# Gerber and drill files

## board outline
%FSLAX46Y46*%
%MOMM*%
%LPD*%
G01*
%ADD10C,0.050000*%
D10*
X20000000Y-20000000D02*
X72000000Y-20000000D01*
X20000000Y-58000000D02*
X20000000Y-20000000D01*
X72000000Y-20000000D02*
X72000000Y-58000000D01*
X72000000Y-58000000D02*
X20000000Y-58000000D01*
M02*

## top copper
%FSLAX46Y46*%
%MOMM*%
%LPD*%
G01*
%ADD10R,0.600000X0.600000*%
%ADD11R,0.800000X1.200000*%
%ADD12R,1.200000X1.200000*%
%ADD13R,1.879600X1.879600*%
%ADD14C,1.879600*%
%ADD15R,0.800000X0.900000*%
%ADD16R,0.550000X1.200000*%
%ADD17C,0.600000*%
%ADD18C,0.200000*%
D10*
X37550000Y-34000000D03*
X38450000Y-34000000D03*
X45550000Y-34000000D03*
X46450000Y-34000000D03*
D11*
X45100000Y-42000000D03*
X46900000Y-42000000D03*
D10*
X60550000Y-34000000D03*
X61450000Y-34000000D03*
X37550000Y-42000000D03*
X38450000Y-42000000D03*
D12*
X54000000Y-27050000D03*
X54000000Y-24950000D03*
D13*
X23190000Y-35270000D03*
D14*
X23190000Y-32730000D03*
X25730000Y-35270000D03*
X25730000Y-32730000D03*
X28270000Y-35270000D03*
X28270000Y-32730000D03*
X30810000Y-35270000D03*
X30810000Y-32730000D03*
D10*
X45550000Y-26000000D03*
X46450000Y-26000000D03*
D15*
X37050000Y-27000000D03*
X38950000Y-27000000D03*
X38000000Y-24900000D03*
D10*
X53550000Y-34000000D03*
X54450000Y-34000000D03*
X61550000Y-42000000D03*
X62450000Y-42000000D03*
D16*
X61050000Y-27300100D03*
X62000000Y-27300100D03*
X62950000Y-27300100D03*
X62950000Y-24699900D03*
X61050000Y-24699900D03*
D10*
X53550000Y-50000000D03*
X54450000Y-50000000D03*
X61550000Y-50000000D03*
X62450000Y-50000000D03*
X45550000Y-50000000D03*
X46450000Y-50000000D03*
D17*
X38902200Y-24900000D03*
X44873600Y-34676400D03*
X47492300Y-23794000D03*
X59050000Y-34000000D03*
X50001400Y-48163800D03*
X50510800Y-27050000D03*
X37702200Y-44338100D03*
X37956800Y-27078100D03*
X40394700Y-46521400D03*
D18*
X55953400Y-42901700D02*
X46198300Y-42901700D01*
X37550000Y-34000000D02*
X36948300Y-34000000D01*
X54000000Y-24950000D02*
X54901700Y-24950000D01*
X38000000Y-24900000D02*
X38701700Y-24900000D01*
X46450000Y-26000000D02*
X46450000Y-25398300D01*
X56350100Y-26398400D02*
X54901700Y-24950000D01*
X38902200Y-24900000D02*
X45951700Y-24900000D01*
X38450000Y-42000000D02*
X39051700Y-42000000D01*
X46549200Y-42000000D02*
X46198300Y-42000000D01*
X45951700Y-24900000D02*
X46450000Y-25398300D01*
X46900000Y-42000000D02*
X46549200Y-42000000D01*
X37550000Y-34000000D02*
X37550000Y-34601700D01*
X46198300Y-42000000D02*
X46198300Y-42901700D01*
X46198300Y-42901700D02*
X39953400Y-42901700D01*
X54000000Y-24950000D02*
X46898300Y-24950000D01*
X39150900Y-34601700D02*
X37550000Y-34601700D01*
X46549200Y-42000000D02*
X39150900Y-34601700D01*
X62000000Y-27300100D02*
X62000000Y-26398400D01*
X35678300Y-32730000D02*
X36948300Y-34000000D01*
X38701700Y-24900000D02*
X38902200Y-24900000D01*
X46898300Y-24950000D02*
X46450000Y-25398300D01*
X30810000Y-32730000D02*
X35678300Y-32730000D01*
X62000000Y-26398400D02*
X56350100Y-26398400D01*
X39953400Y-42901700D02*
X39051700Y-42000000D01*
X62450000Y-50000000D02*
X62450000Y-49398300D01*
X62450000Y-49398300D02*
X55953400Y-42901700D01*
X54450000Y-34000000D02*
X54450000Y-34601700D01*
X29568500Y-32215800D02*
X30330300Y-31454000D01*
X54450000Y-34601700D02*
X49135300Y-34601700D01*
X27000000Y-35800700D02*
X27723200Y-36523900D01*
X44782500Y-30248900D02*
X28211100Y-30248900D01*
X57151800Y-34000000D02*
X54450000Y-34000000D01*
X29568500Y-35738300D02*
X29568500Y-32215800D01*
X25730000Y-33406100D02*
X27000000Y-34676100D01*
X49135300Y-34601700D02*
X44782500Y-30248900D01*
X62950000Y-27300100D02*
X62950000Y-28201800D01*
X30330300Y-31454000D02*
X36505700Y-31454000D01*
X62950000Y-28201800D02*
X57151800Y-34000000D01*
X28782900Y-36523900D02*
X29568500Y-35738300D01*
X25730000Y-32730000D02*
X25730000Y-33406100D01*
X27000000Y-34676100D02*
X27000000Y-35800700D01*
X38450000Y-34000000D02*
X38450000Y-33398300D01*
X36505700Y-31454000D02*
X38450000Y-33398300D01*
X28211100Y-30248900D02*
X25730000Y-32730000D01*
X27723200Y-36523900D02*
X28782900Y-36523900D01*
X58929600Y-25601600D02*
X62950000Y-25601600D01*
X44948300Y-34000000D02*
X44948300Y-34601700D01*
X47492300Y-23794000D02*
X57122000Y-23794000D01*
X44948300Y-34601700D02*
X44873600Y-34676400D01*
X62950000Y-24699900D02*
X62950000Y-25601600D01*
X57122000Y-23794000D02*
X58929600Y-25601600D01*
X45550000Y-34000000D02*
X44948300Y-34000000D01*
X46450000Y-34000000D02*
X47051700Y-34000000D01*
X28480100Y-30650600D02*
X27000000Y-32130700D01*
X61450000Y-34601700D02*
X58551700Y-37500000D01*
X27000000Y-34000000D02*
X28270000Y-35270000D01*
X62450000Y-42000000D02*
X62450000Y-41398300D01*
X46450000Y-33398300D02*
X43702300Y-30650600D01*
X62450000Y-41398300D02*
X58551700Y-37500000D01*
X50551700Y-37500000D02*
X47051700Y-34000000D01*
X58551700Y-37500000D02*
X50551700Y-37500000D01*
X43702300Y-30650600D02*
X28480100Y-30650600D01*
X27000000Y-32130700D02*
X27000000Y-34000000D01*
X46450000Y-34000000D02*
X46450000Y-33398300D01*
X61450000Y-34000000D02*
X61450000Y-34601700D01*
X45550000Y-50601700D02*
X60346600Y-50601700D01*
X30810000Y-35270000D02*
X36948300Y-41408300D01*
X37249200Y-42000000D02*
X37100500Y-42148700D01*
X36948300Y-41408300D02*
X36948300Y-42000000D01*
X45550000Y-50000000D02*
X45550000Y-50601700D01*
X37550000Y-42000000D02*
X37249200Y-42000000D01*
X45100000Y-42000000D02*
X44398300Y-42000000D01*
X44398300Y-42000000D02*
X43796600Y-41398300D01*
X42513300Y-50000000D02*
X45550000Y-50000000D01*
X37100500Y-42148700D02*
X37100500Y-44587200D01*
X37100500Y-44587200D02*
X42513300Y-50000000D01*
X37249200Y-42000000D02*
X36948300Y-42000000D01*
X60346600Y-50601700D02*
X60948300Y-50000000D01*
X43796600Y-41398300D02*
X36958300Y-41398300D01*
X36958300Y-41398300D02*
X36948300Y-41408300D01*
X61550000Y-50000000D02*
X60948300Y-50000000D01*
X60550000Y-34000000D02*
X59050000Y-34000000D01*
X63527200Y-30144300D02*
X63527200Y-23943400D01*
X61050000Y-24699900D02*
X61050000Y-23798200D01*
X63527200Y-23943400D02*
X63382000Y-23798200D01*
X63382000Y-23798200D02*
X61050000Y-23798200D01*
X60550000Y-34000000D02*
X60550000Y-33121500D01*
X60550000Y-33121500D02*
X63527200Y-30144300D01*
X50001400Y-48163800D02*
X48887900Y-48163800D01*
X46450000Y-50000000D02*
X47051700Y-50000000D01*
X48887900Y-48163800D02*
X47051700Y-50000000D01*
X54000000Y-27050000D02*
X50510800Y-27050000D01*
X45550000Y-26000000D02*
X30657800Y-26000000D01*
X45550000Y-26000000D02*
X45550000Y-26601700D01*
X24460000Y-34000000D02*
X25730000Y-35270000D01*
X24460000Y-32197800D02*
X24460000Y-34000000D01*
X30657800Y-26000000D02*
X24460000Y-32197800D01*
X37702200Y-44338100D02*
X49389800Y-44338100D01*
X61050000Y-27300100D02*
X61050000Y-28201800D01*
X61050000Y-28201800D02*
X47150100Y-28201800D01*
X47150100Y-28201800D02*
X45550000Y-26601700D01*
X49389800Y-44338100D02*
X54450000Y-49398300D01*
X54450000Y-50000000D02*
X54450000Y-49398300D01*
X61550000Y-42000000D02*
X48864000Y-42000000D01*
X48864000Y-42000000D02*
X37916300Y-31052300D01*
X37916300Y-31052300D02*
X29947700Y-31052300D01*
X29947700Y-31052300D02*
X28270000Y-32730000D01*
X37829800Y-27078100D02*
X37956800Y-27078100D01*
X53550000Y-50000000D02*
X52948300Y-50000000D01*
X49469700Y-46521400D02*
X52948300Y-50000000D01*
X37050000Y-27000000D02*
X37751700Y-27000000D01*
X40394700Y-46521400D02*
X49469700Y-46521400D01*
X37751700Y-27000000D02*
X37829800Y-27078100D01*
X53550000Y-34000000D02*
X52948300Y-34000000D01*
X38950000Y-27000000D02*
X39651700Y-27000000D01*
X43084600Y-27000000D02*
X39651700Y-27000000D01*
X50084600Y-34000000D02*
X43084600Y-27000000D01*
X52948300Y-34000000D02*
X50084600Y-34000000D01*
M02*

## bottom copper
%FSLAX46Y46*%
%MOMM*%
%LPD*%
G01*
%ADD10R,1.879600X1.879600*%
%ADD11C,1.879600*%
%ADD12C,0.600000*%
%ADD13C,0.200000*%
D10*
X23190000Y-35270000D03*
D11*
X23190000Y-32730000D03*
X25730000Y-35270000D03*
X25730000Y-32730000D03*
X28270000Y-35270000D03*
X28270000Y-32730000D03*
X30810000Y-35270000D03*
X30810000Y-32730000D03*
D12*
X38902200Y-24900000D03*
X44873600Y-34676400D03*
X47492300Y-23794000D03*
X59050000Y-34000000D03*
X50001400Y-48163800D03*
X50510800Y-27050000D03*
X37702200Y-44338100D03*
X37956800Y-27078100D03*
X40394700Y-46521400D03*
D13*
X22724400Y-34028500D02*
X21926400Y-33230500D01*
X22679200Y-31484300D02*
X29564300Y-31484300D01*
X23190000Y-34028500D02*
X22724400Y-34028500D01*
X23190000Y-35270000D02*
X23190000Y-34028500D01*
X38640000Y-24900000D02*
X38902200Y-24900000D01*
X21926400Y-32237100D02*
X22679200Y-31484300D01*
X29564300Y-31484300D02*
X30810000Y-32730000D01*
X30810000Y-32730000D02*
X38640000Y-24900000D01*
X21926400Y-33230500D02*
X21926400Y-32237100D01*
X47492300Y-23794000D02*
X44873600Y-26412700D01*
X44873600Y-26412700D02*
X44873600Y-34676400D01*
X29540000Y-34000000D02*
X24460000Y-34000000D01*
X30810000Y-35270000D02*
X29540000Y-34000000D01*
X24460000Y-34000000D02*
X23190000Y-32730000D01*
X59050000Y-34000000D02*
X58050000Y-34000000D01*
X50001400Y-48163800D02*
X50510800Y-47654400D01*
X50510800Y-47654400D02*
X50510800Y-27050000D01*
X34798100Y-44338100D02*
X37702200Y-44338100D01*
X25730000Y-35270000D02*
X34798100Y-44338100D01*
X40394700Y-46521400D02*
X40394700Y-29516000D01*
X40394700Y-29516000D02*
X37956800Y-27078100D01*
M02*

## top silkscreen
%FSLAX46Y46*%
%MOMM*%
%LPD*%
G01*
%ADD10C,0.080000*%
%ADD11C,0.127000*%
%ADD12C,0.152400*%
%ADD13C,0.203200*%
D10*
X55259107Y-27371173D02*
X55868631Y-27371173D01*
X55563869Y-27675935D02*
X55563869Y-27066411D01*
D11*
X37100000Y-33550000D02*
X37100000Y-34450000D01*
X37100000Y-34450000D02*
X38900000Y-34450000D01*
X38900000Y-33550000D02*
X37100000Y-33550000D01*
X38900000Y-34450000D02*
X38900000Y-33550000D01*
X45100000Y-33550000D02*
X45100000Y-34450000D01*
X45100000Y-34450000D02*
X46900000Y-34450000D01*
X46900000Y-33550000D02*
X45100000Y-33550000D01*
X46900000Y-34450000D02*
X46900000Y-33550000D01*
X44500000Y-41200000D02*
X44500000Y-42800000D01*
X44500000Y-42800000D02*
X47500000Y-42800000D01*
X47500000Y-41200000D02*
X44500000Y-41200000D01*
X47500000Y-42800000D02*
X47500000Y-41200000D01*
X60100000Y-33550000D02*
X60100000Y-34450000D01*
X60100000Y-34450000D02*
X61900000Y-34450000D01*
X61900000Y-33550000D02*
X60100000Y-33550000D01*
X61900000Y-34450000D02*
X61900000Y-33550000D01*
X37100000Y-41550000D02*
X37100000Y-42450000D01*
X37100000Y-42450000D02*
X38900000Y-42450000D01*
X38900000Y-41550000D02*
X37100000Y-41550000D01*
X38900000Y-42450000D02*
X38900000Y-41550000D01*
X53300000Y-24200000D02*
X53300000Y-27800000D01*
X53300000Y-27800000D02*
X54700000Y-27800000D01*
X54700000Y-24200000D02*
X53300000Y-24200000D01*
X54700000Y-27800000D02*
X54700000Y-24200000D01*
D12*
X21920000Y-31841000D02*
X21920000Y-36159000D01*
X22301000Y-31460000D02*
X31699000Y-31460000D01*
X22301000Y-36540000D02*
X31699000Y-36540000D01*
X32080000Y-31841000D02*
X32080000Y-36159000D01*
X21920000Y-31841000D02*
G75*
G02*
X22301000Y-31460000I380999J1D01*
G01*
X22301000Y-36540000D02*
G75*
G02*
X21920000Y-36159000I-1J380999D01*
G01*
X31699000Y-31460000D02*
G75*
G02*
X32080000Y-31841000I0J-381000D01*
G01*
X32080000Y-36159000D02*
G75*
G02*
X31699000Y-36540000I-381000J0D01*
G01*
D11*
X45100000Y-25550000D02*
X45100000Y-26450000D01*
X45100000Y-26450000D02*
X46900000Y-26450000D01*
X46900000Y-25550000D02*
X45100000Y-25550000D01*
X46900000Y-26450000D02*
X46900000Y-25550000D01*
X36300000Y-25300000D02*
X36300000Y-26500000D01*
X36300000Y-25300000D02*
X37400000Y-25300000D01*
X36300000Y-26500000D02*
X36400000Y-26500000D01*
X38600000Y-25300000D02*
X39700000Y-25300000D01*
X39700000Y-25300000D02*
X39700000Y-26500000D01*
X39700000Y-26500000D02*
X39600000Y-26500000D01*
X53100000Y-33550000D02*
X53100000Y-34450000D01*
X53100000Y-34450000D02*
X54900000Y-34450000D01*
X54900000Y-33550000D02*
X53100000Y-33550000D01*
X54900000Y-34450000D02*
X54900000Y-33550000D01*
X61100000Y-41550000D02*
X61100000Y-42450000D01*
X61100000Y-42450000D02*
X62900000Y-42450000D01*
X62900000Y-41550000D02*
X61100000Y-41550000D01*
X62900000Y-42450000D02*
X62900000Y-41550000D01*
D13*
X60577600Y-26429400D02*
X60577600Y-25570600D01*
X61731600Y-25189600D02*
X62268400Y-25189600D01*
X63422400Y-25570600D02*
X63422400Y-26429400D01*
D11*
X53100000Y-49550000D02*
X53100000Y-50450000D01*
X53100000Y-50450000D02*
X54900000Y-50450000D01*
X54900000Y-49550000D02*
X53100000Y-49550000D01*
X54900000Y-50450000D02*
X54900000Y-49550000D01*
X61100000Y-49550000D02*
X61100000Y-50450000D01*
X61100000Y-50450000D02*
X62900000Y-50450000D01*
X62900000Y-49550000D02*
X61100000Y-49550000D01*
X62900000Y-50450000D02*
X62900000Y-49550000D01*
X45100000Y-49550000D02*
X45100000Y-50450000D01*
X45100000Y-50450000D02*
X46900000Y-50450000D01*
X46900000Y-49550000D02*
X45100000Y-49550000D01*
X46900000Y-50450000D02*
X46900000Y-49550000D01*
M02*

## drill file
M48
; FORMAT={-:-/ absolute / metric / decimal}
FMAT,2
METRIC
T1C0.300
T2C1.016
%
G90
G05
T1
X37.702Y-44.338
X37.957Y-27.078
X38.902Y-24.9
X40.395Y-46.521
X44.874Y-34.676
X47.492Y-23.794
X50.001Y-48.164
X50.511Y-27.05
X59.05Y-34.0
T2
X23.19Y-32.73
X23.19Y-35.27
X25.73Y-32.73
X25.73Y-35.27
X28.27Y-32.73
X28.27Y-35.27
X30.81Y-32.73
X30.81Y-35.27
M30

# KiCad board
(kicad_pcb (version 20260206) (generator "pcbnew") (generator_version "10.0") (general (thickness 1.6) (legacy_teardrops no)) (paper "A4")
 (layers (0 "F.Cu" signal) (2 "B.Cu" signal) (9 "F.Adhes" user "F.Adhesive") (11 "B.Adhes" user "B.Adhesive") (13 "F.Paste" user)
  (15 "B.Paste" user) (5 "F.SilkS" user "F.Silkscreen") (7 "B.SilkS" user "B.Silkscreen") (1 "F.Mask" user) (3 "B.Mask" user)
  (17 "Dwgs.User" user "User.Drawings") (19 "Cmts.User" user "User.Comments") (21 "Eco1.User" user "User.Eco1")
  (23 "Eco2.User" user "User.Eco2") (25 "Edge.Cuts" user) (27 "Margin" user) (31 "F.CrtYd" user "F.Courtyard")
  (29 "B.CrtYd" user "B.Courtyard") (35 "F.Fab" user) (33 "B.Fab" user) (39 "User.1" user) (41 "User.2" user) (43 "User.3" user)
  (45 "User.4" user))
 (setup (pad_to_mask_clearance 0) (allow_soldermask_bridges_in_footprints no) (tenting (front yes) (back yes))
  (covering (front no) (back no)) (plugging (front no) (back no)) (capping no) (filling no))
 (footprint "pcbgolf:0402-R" (layer "F.Cu") (at 38 34)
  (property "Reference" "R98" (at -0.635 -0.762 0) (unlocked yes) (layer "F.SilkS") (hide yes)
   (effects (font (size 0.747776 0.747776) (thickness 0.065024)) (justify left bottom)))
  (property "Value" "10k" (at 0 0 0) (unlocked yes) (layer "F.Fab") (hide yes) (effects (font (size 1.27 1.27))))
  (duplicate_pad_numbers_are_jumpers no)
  (fp_line (start -0.9 -0.45) (end -0.9 0.45) (stroke (width 0.127) (type solid)) (layer "F.SilkS"))
  (fp_line (start -0.9 0.45) (end 0.9 0.45) (stroke (width 0.127) (type solid)) (layer "F.SilkS"))
  (fp_line (start 0.9 -0.45) (end -0.9 -0.45) (stroke (width 0.127) (type solid)) (layer "F.SilkS"))
  (fp_line (start 0.9 0.45) (end 0.9 -0.45) (stroke (width 0.127) (type solid)) (layer "F.SilkS"))
  (pad "1" smd rect (at -0.45 0) (size 0.6 0.6) (layers "F.Cu" "F.Mask" "F.Paste") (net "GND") (solder_mask_margin 0.0508)
   (solder_paste_margin 0) (thermal_bridge_angle 0))
  (pad "2" smd rect (at 0.45 0) (size 0.6 0.6) (layers "F.Cu" "F.Mask" "F.Paste") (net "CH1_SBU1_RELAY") (solder_mask_margin 0.0508)
   (solder_paste_margin 0) (thermal_bridge_angle 0)))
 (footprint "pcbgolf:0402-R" (layer "F.Cu") (at 46 34)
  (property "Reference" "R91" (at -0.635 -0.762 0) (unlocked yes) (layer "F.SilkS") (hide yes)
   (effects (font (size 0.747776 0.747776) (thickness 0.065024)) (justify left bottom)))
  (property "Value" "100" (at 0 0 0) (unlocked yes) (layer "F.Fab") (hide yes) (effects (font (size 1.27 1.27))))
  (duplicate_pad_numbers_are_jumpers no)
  (fp_line (start -0.9 -0.45) (end -0.9 0.45) (stroke (width 0.127) (type solid)) (layer "F.SilkS"))
  (fp_line (start -0.9 0.45) (end 0.9 0.45) (stroke (width 0.127) (type solid)) (layer "F.SilkS"))
  (fp_line (start 0.9 -0.45) (end -0.9 -0.45) (stroke (width 0.127) (type solid)) (layer "F.SilkS"))
  (fp_line (start 0.9 0.45) (end 0.9 -0.45) (stroke (width 0.127) (type solid)) (layer "F.SilkS"))
  (pad "1" smd rect (at -0.45 0) (size 0.6 0.6) (layers "F.Cu" "F.Mask" "F.Paste") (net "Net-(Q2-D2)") (solder_mask_margin 0.0508)
   (solder_paste_margin 0) (thermal_bridge_angle 0))
  (pad "2" smd rect (at 0.45 0) (size 0.6 0.6) (layers "F.Cu" "F.Mask" "F.Paste") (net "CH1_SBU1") (solder_mask_margin 0.0508)
   (solder_paste_margin 0) (thermal_bridge_angle 0)))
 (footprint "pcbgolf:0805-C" (layer "F.Cu") (at 46 42)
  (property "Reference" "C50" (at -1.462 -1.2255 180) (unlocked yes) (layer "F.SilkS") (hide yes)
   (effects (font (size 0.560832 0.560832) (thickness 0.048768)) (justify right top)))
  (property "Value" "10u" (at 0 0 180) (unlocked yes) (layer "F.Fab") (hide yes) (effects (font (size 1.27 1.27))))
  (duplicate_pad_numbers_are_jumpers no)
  (fp_line (start -1.5 -0.8) (end -1.5 0.8) (stroke (width 0.127) (type solid)) (layer "F.SilkS"))
  (fp_line (start -1.5 0.8) (end 1.5 0.8) (stroke (width 0.127) (type solid)) (layer "F.SilkS"))
  (fp_line (start 1.5 -0.8) (end -1.5 -0.8) (stroke (width 0.127) (type solid)) (layer "F.SilkS"))
  (fp_line (start 1.5 0.8) (end 1.5 -0.8) (stroke (width 0.127) (type solid)) (layer "F.SilkS"))
  (pad "1" smd rect (at -0.9 0) (size 0.8 1.2) (layers "F.Cu" "F.Mask" "F.Paste") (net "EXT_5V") (solder_mask_margin 0.0508)
   (solder_paste_margin 0) (thermal_bridge_angle 0))
  (pad "2" smd rect (at 0.9 0) (size 0.8 1.2) (layers "F.Cu" "F.Mask" "F.Paste") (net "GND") (solder_mask_margin 0.0508)
   (solder_paste_margin 0) (thermal_bridge_angle 0)))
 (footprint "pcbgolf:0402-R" (layer "F.Cu") (at 61 34)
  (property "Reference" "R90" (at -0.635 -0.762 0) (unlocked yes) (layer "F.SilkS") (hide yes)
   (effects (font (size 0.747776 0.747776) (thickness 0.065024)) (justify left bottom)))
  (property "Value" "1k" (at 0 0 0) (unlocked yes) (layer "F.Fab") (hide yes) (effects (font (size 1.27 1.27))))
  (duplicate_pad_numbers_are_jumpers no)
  (fp_line (start -0.9 -0.45) (end -0.9 0.45) (stroke (width 0.127) (type solid)) (layer "F.SilkS"))
  (fp_line (start -0.9 0.45) (end 0.9 0.45) (stroke (width 0.127) (type solid)) (layer "F.SilkS"))
  (fp_line (start 0.9 -0.45) (end -0.9 -0.45) (stroke (width 0.127) (type solid)) (layer "F.SilkS"))
  (fp_line (start 0.9 0.45) (end 0.9 -0.45) (stroke (width 0.127) (type solid)) (layer "F.SilkS"))
  (pad "1" smd rect (at -0.45 0) (size 0.6 0.6) (layers "F.Cu" "F.Mask" "F.Paste") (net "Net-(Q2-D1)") (solder_mask_margin 0.0508)
   (solder_paste_margin 0) (thermal_bridge_angle 0))
  (pad "2" smd rect (at 0.45 0) (size 0.6 0.6) (layers "F.Cu" "F.Mask" "F.Paste") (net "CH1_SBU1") (solder_mask_margin 0.0508)
   (solder_paste_margin 0) (thermal_bridge_angle 0)))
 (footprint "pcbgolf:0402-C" (layer "F.Cu") (at 38 42)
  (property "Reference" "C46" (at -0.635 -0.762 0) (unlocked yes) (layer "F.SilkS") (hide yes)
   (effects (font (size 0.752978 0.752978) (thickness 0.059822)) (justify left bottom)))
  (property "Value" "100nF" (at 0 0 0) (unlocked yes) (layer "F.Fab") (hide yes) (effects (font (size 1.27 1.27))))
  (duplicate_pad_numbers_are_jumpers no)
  (fp_line (start -0.9 -0.45) (end -0.9 0.45) (stroke (width 0.127) (type solid)) (layer "F.SilkS"))
  (fp_line (start -0.9 0.45) (end 0.9 0.45) (stroke (width 0.127) (type solid)) (layer "F.SilkS"))
  (fp_line (start 0.9 -0.45) (end -0.9 -0.45) (stroke (width 0.127) (type solid)) (layer "F.SilkS"))
  (fp_line (start 0.9 0.45) (end 0.9 -0.45) (stroke (width 0.127) (type solid)) (layer "F.SilkS"))
  (pad "1" smd rect (at -0.45 0) (size 0.6 0.6) (layers "F.Cu" "F.Mask" "F.Paste") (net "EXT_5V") (solder_mask_margin 0.0508)
   (solder_paste_margin 0) (thermal_bridge_angle 0))
  (pad "2" smd rect (at 0.45 0) (size 0.6 0.6) (layers "F.Cu" "F.Mask" "F.Paste") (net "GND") (solder_mask_margin 0.0508)
   (solder_paste_margin 0) (thermal_bridge_angle 0)))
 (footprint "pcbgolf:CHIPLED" (layer "F.Cu") (at 54 26)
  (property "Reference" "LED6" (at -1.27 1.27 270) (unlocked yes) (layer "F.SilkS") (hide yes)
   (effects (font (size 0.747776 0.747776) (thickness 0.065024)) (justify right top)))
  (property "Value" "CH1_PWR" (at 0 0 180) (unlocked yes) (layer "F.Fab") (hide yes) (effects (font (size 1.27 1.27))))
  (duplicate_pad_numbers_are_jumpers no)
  (fp_line (start -0.7 -1.8) (end -0.7 1.8) (stroke (width 0.127) (type solid)) (layer "F.SilkS"))
  (fp_line (start -0.7 1.8) (end 0.7 1.8) (stroke (width 0.127) (type solid)) (layer "F.SilkS"))
  (fp_line (start 0.7 -1.8) (end -0.7 -1.8) (stroke (width 0.127) (type solid)) (layer "F.SilkS"))
  (fp_line (start 0.7 1.8) (end 0.7 -1.8) (stroke (width 0.127) (type solid)) (layer "F.SilkS"))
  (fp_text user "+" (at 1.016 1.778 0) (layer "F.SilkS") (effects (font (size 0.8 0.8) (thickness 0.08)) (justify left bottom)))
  (pad "A" smd rect (at 0 1.05) (size 1.2 1.2) (layers "F.Cu" "F.Mask" "F.Paste") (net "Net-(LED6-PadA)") (solder_mask_margin 0.0508)
   (solder_paste_margin 0) (thermal_bridge_angle 0))
  (pad "C" smd rect (at 0 -1.05) (size 1.2 1.2) (layers "F.Cu" "F.Mask" "F.Paste") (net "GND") (solder_mask_margin 0.0508)
   (solder_paste_margin 0) (thermal_bridge_angle 0)))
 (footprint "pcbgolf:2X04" (layer "F.Cu") (at 27 34)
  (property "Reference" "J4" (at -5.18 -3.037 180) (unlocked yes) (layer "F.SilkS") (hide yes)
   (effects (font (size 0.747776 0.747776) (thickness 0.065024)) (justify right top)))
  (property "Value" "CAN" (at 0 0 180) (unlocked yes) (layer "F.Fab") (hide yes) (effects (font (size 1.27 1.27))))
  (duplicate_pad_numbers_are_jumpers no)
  (fp_line (start -5.08 -2.159) (end -5.08 2.159) (stroke (width 0.1524) (type solid)) (layer "F.SilkS"))
  (fp_line (start -4.699 -2.54) (end 4.699 -2.54) (stroke (width 0.1524) (type solid)) (layer "F.SilkS"))
  (fp_line (start -4.699 2.54) (end 4.699 2.54) (stroke (width 0.1524) (type solid)) (layer "F.SilkS"))
  (fp_line (start 5.08 -2.159) (end 5.08 2.159) (stroke (width 0.1524) (type solid)) (layer "F.SilkS"))
  (fp_arc (start -5.08 -2.159) (mid -4.968408 -2.428408) (end -4.699 -2.54) (stroke (width 0.1524) (type solid)) (layer "F.SilkS"))
  (fp_arc (start -4.699 2.54) (mid -4.968408 2.428408) (end -5.08 2.159) (stroke (width 0.1524) (type solid)) (layer "F.SilkS"))
  (fp_arc (start 4.699 -2.54) (mid 4.968408 -2.428408) (end 5.08 -2.159) (stroke (width 0.1524) (type solid)) (layer "F.SilkS"))
  (fp_arc (start 5.08 2.159) (mid 4.968408 2.428408) (end 4.699 2.54) (stroke (width 0.1524) (type solid)) (layer "F.SilkS"))
  (pad "1" thru_hole rect (at -3.81 1.27 90) (size 1.8796 1.8796) (drill 1.016) (layers "*.Cu" "*.Mask") (remove_unused_layers no)
   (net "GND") (solder_mask_margin 0.0508) (thermal_bridge_angle 0))
  (pad "2" thru_hole circle (at -3.81 -1.27 90) (size 1.8796 1.8796) (drill 1.016) (layers "*.Cu" "*.Mask") (remove_unused_layers no)
   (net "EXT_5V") (solder_mask_margin 0.0508) (thermal_bridge_angle 0))
  (pad "3" thru_hole circle (at -1.27 1.27 90) (size 1.8796 1.8796) (drill 1.016) (layers "*.Cu" "*.Mask") (remove_unused_layers no)
   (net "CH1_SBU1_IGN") (solder_mask_margin 0.0508) (thermal_bridge_angle 0))
  (pad "4" thru_hole circle (at -1.27 -1.27 90) (size 1.8796 1.8796) (drill 1.016) (layers "*.Cu" "*.Mask") (remove_unused_layers no)
   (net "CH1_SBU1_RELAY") (solder_mask_margin 0.0508) (thermal_bridge_angle 0))
  (pad "5" thru_hole circle (at 1.27 1.27 90) (size 1.8796 1.8796) (drill 1.016) (layers "*.Cu" "*.Mask") (remove_unused_layers no)
   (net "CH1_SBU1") (solder_mask_margin 0.0508) (thermal_bridge_angle 0))
  (pad "6" thru_hole circle (at 1.27 -1.27 90) (size 1.8796 1.8796) (drill 1.016) (layers "*.Cu" "*.Mask") (remove_unused_layers no)
   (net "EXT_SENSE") (solder_mask_margin 0.0508) (thermal_bridge_angle 0))
  (pad "7" thru_hole circle (at 3.81 1.27 90) (size 1.8796 1.8796) (drill 1.016) (layers "*.Cu" "*.Mask") (remove_unused_layers no)
   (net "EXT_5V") (solder_mask_margin 0.0508) (thermal_bridge_angle 0))
  (pad "8" thru_hole circle (at 3.81 -1.27 90) (size 1.8796 1.8796) (drill 1.016) (layers "*.Cu" "*.Mask") (remove_unused_layers no)
   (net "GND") (solder_mask_margin 0.0508) (thermal_bridge_angle 0)))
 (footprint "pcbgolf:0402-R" (layer "F.Cu") (at 46 26)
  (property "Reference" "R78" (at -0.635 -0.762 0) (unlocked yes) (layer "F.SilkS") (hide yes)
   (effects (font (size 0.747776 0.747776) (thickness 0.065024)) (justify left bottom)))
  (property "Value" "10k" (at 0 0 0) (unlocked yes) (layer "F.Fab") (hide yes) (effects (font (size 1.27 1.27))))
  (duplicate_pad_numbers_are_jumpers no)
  (fp_line (start -0.9 -0.45) (end -0.9 0.45) (stroke (width 0.127) (type solid)) (layer "F.SilkS"))
  (fp_line (start -0.9 0.45) (end 0.9 0.45) (stroke (width 0.127) (type solid)) (layer "F.SilkS"))
  (fp_line (start 0.9 -0.45) (end -0.9 -0.45) (stroke (width 0.127) (type solid)) (layer "F.SilkS"))
  (fp_line (start 0.9 0.45) (end 0.9 -0.45) (stroke (width 0.127) (type solid)) (layer "F.SilkS"))
  (pad "1" smd rect (at -0.45 0) (size 0.6 0.6) (layers "F.Cu" "F.Mask" "F.Paste") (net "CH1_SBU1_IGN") (solder_mask_margin 0.0508)
   (solder_paste_margin 0) (thermal_bridge_angle 0))
  (pad "2" smd rect (at 0.45 0) (size 0.6 0.6) (layers "F.Cu" "F.Mask" "F.Paste") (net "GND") (solder_mask_margin 0.0508)
   (solder_paste_margin 0) (thermal_bridge_angle 0)))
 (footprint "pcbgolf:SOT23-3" (layer "F.Cu") (at 38 26)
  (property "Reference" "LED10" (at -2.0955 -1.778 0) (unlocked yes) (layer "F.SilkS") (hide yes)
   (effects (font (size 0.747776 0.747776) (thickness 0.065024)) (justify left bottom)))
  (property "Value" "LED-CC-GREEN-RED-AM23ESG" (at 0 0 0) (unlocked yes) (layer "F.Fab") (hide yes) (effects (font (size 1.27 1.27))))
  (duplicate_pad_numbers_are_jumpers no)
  (fp_line (start -1.7 -0.7) (end -1.7 0.5) (stroke (width 0.127) (type solid)) (layer "F.SilkS"))
  (fp_line (start -1.7 -0.7) (end -0.6 -0.7) (stroke (width 0.127) (type solid)) (layer "F.SilkS"))
  (fp_line (start -1.7 0.5) (end -1.6 0.5) (stroke (width 0.127) (type solid)) (layer "F.SilkS"))
  (fp_line (start 0.6 -0.7) (end 1.7 -0.7) (stroke (width 0.127) (type solid)) (layer "F.SilkS"))
  (fp_line (start 1.7 -0.7) (end 1.7 0.5) (stroke (width 0.127) (type solid)) (layer "F.SilkS"))
  (fp_line (start 1.7 0.5) (end 1.6 0.5) (stroke (width 0.127) (type solid)) (layer "F.SilkS"))
  (pad "1" smd rect (at -0.95 1) (size 0.8 0.9) (layers "F.Cu" "F.Mask" "F.Paste") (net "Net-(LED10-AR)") (solder_mask_margin 0.0508)
   (solder_paste_margin 0) (thermal_bridge_angle 0))
  (pad "2" smd rect (at 0.95 1) (size 0.8 0.9) (layers "F.Cu" "F.Mask" "F.Paste") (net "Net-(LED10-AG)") (solder_mask_margin 0.0508)
   (solder_paste_margin 0) (thermal_bridge_angle 0))
  (pad "3" smd rect (at 0 -1.1) (size 0.8 0.9) (layers "F.Cu" "F.Mask" "F.Paste") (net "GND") (solder_mask_margin 0.0508)
   (solder_paste_margin 0) (thermal_bridge_angle 0)))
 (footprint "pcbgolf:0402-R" (layer "F.Cu") (at 54 34)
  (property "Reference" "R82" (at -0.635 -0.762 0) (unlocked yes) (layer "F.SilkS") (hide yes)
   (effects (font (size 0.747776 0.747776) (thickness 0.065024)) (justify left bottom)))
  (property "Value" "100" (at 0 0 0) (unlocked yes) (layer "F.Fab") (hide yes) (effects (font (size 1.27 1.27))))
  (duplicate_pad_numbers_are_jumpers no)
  (fp_line (start -0.9 -0.45) (end -0.9 0.45) (stroke (width 0.127) (type solid)) (layer "F.SilkS"))
  (fp_line (start -0.9 0.45) (end 0.9 0.45) (stroke (width 0.127) (type solid)) (layer "F.SilkS"))
  (fp_line (start 0.9 -0.45) (end -0.9 -0.45) (stroke (width 0.127) (type solid)) (layer "F.SilkS"))
  (fp_line (start 0.9 0.45) (end 0.9 -0.45) (stroke (width 0.127) (type solid)) (layer "F.SilkS"))
  (pad "1" smd rect (at -0.45 0) (size 0.6 0.6) (layers "F.Cu" "F.Mask" "F.Paste") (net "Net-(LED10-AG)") (solder_mask_margin 0.0508)
   (solder_paste_margin 0) (thermal_bridge_angle 0))
  (pad "2" smd rect (at 0.45 0) (size 0.6 0.6) (layers "F.Cu" "F.Mask" "F.Paste") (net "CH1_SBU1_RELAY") (solder_mask_margin 0.0508)
   (solder_paste_margin 0) (thermal_bridge_angle 0)))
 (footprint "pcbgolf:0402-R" (layer "F.Cu") (at 62 42)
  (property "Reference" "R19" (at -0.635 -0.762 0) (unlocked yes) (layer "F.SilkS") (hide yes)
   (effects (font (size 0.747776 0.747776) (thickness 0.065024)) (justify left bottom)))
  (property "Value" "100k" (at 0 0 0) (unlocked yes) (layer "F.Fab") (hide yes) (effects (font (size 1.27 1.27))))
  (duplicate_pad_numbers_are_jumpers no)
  (fp_line (start -0.9 -0.45) (end -0.9 0.45) (stroke (width 0.127) (type solid)) (layer "F.SilkS"))
  (fp_line (start -0.9 0.45) (end 0.9 0.45) (stroke (width 0.127) (type solid)) (layer "F.SilkS"))
  (fp_line (start 0.9 -0.45) (end -0.9 -0.45) (stroke (width 0.127) (type solid)) (layer "F.SilkS"))
  (fp_line (start 0.9 0.45) (end 0.9 -0.45) (stroke (width 0.127) (type solid)) (layer "F.SilkS"))
  (pad "1" smd rect (at -0.45 0) (size 0.6 0.6) (layers "F.Cu" "F.Mask" "F.Paste") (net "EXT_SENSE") (solder_mask_margin 0.0508)
   (solder_paste_margin 0) (thermal_bridge_angle 0))
  (pad "2" smd rect (at 0.45 0) (size 0.6 0.6) (layers "F.Cu" "F.Mask" "F.Paste") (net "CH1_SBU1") (solder_mask_margin 0.0508)
   (solder_paste_margin 0) (thermal_bridge_angle 0)))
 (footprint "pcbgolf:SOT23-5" (layer "F.Cu") (at 62 26)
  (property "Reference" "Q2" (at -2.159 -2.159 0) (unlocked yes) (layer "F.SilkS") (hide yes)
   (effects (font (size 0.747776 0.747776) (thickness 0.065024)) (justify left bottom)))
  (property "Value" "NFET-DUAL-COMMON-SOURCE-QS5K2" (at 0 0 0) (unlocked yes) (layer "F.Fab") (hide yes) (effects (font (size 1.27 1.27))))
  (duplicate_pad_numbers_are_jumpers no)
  (fp_line (start -1.4224 0.4294) (end -1.4224 -0.4294) (stroke (width 0.2032) (type solid)) (layer "F.SilkS"))
  (fp_line (start -0.2684 -0.8104) (end 0.2684 -0.8104) (stroke (width 0.2032) (type solid)) (layer "F.SilkS"))
  (fp_line (start 1.4224 -0.4294) (end 1.4224 0.4294) (stroke (width 0.2032) (type solid)) (layer "F.SilkS"))
  (pad "1" smd rect (at -0.95 1.3001) (size 0.55 1.2) (layers "F.Cu" "F.Mask" "F.Paste") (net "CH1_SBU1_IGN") (solder_mask_margin 0.0508)
   (solder_paste_margin 0) (thermal_bridge_angle 0))
  (pad "2" smd rect (at 0 1.3001) (size 0.55 1.2) (layers "F.Cu" "F.Mask" "F.Paste") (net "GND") (solder_mask_margin 0.0508)
   (solder_paste_margin 0) (thermal_bridge_angle 0))
  (pad "3" smd rect (at 0.95 1.3001) (size 0.55 1.2) (layers "F.Cu" "F.Mask" "F.Paste") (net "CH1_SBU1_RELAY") (solder_mask_margin 0.0508)
   (solder_paste_margin 0) (thermal_bridge_angle 0))
  (pad "4" smd rect (at 0.95 -1.3001) (size 0.55 1.2) (layers "F.Cu" "F.Mask" "F.Paste") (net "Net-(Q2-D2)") (solder_mask_margin 0.0508)
   (solder_paste_margin 0) (thermal_bridge_angle 0))
  (pad "5" smd rect (at -0.95 -1.3001) (size 0.55 1.2) (layers "F.Cu" "F.Mask" "F.Paste") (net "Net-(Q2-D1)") (solder_mask_margin 0.0508)
   (solder_paste_margin 0) (thermal_bridge_angle 0)))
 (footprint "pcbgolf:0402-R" (layer "F.Cu") (at 54 50)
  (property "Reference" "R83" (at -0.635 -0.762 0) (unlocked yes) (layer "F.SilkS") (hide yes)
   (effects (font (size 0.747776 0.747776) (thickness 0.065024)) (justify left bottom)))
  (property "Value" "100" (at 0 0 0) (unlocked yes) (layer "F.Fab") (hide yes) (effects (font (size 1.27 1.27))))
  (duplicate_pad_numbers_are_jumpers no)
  (fp_line (start -0.9 -0.45) (end -0.9 0.45) (stroke (width 0.127) (type solid)) (layer "F.SilkS"))
  (fp_line (start -0.9 0.45) (end 0.9 0.45) (stroke (width 0.127) (type solid)) (layer "F.SilkS"))
  (fp_line (start 0.9 -0.45) (end -0.9 -0.45) (stroke (width 0.127) (type solid)) (layer "F.SilkS"))
  (fp_line (start 0.9 0.45) (end 0.9 -0.45) (stroke (width 0.127) (type solid)) (layer "F.SilkS"))
  (pad "1" smd rect (at -0.45 0) (size 0.6 0.6) (layers "F.Cu" "F.Mask" "F.Paste") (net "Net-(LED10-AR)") (solder_mask_margin 0.0508)
   (solder_paste_margin 0) (thermal_bridge_angle 0))
  (pad "2" smd rect (at 0.45 0) (size 0.6 0.6) (layers "F.Cu" "F.Mask" "F.Paste") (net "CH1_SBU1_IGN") (solder_mask_margin 0.0508)
   (solder_paste_margin 0) (thermal_bridge_angle 0)))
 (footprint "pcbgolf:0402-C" (layer "F.Cu") (at 62 50)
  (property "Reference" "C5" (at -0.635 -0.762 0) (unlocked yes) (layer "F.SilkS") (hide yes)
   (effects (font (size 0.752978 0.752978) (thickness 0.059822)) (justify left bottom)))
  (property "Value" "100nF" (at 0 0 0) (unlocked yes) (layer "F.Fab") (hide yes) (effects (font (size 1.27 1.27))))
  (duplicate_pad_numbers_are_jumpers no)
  (fp_line (start -0.9 -0.45) (end -0.9 0.45) (stroke (width 0.127) (type solid)) (layer "F.SilkS"))
  (fp_line (start -0.9 0.45) (end 0.9 0.45) (stroke (width 0.127) (type solid)) (layer "F.SilkS"))
  (fp_line (start 0.9 -0.45) (end -0.9 -0.45) (stroke (width 0.127) (type solid)) (layer "F.SilkS"))
  (fp_line (start 0.9 0.45) (end 0.9 -0.45) (stroke (width 0.127) (type solid)) (layer "F.SilkS"))
  (pad "1" smd rect (at -0.45 0) (size 0.6 0.6) (layers "F.Cu" "F.Mask" "F.Paste") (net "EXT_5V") (solder_mask_margin 0.0508)
   (solder_paste_margin 0) (thermal_bridge_angle 0))
  (pad "2" smd rect (at 0.45 0) (size 0.6 0.6) (layers "F.Cu" "F.Mask" "F.Paste") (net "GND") (solder_mask_margin 0.0508)
   (solder_paste_margin 0) (thermal_bridge_angle 0)))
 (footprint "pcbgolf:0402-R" (layer "F.Cu") (at 46 50)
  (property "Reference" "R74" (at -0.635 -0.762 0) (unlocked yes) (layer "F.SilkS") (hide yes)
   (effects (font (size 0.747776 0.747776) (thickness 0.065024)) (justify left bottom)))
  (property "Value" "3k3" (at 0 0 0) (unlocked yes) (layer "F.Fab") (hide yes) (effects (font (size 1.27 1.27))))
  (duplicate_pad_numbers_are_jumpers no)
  (fp_line (start -0.9 -0.45) (end -0.9 0.45) (stroke (width 0.127) (type solid)) (layer "F.SilkS"))
  (fp_line (start -0.9 0.45) (end 0.9 0.45) (stroke (width 0.127) (type solid)) (layer "F.SilkS"))
  (fp_line (start 0.9 -0.45) (end -0.9 -0.45) (stroke (width 0.127) (type solid)) (layer "F.SilkS"))
  (fp_line (start 0.9 0.45) (end 0.9 -0.45) (stroke (width 0.127) (type solid)) (layer "F.SilkS"))
  (pad "1" smd rect (at -0.45 0) (size 0.6 0.6) (layers "F.Cu" "F.Mask" "F.Paste") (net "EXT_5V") (solder_mask_margin 0.0508)
   (solder_paste_margin 0) (thermal_bridge_angle 0))
  (pad "2" smd rect (at 0.45 0) (size 0.6 0.6) (layers "F.Cu" "F.Mask" "F.Paste") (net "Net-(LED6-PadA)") (solder_mask_margin 0.0508)
   (solder_paste_margin 0) (thermal_bridge_angle 0)))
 (gr_line (start 20 20) (end 72 20) (stroke (width 0.05) (type default)) (layer "Edge.Cuts"))
 (gr_line (start 20 58) (end 20 20) (stroke (width 0.05) (type default)) (layer "Edge.Cuts"))
 (gr_line (start 72 20) (end 72 58) (stroke (width 0.05) (type default)) (layer "Edge.Cuts"))
 (gr_line (start 72 58) (end 20 58) (stroke (width 0.05) (type default)) (layer "Edge.Cuts"))
 (segment (start 55.9534 42.9017) (end 46.1983 42.9017) (width 0.2) (layer "F.Cu") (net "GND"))
 (segment (start 37.55 34) (end 36.9483 34) (width 0.2) (layer "F.Cu") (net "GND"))
 (segment (start 54 24.95) (end 54.9017 24.95) (width 0.2) (layer "F.Cu") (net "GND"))
 (segment (start 38 24.9) (end 38.7017 24.9) (width 0.2) (layer "F.Cu") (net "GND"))
 (segment (start 46.45 26) (end 46.45 25.3983) (width 0.2) (layer "F.Cu") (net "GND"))
 (segment (start 56.3501 26.3984) (end 54.9017 24.95) (width 0.2) (layer "F.Cu") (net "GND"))
 (segment (start 38.9022 24.9) (end 45.9517 24.9) (width 0.2) (layer "F.Cu") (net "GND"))
 (segment (start 38.45 42) (end 39.0517 42) (width 0.2) (layer "F.Cu") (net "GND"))
 (segment (start 46.5492 42) (end 46.1983 42) (width 0.2) (layer "F.Cu") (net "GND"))
 (segment (start 45.9517 24.9) (end 46.45 25.3983) (width 0.2) (layer "F.Cu") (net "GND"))
 (segment (start 46.9 42) (end 46.5492 42) (width 0.2) (layer "F.Cu") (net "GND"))
 (segment (start 37.55 34) (end 37.55 34.6017) (width 0.2) (layer "F.Cu") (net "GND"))
 (segment (start 46.1983 42) (end 46.1983 42.9017) (width 0.2) (layer "F.Cu") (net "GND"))
 (segment (start 46.1983 42.9017) (end 39.9534 42.9017) (width 0.2) (layer "F.Cu") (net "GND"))
 (segment (start 54 24.95) (end 46.8983 24.95) (width 0.2) (layer "F.Cu") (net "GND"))
 (segment (start 39.1509 34.6017) (end 37.55 34.6017) (width 0.2) (layer "F.Cu") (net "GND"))
 (segment (start 46.5492 42) (end 39.1509 34.6017) (width 0.2) (layer "F.Cu") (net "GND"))
 (segment (start 62 27.3001) (end 62 26.3984) (width 0.2) (layer "F.Cu") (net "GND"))
 (segment (start 35.6783 32.73) (end 36.9483 34) (width 0.2) (layer "F.Cu") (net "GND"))
 (segment (start 38.7017 24.9) (end 38.9022 24.9) (width 0.2) (layer "F.Cu") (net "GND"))
 (segment (start 46.8983 24.95) (end 46.45 25.3983) (width 0.2) (layer "F.Cu") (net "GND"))
 (segment (start 30.81 32.73) (end 35.6783 32.73) (width 0.2) (layer "F.Cu") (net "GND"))
 (segment (start 62 26.3984) (end 56.3501 26.3984) (width 0.2) (layer "F.Cu") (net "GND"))
 (segment (start 39.9534 42.9017) (end 39.0517 42) (width 0.2) (layer "F.Cu") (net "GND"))
 (segment (start 62.45 50) (end 62.45 49.3983) (width 0.2) (layer "F.Cu") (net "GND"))
 (segment (start 62.45 49.3983) (end 55.9534 42.9017) (width 0.2) (layer "F.Cu") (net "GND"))
 (via (at 38.9022 24.9) (size 0.6) (drill 0.3) (layers "F.Cu" "B.Cu") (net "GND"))
 (segment (start 22.7244 34.0285) (end 21.9264 33.2305) (width 0.2) (layer "B.Cu") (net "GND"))
 (segment (start 22.6792 31.4843) (end 29.5643 31.4843) (width 0.2) (layer "B.Cu") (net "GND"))
 (segment (start 23.19 34.0285) (end 22.7244 34.0285) (width 0.2) (layer "B.Cu") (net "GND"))
 (segment (start 23.19 35.27) (end 23.19 34.0285) (width 0.2) (layer "B.Cu") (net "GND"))
 (segment (start 38.64 24.9) (end 38.9022 24.9) (width 0.2) (layer "B.Cu") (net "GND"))
 (segment (start 21.9264 32.2371) (end 22.6792 31.4843) (width 0.2) (layer "B.Cu") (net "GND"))
 (segment (start 29.5643 31.4843) (end 30.81 32.73) (width 0.2) (layer "B.Cu") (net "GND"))
 (segment (start 30.81 32.73) (end 38.64 24.9) (width 0.2) (layer "B.Cu") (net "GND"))
 (segment (start 21.9264 33.2305) (end 21.9264 32.2371) (width 0.2) (layer "B.Cu") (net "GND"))
 (segment (start 54.45 34) (end 54.45 34.6017) (width 0.2) (layer "F.Cu") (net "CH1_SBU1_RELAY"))
 (segment (start 29.5685 32.2158) (end 30.3303 31.454) (width 0.2) (layer "F.Cu") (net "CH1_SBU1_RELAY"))
 (segment (start 54.45 34.6017) (end 49.1353 34.6017) (width 0.2) (layer "F.Cu") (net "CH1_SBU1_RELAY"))
 (segment (start 27 35.8007) (end 27.7232 36.5239) (width 0.2) (layer "F.Cu") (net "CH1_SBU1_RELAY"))
 (segment (start 44.7825 30.2489) (end 28.2111 30.2489) (width 0.2) (layer "F.Cu") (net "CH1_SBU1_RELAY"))
 (segment (start 57.1518 34) (end 54.45 34) (width 0.2) (layer "F.Cu") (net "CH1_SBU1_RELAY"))
 (segment (start 29.5685 35.7383) (end 29.5685 32.2158) (width 0.2) (layer "F.Cu") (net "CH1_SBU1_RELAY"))
 (segment (start 25.73 33.4061) (end 27 34.6761) (width 0.2) (layer "F.Cu") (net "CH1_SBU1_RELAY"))
 (segment (start 49.1353 34.6017) (end 44.7825 30.2489) (width 0.2) (layer "F.Cu") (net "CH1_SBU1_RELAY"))
 (segment (start 62.95 27.3001) (end 62.95 28.2018) (width 0.2) (layer "F.Cu") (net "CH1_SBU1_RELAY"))
 (segment (start 30.3303 31.454) (end 36.5057 31.454) (width 0.2) (layer "F.Cu") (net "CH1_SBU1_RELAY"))
 (segment (start 62.95 28.2018) (end 57.1518 34) (width 0.2) (layer "F.Cu") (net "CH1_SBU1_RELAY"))
 (segment (start 28.7829 36.5239) (end 29.5685 35.7383) (width 0.2) (layer "F.Cu") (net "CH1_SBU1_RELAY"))
 (segment (start 25.73 32.73) (end 25.73 33.4061) (width 0.2) (layer "F.Cu") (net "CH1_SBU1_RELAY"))
 (segment (start 27 34.6761) (end 27 35.8007) (width 0.2) (layer "F.Cu") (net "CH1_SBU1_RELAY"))
 (segment (start 38.45 34) (end 38.45 33.3983) (width 0.2) (layer "F.Cu") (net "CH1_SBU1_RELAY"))
 (segment (start 36.5057 31.454) (end 38.45 33.3983) (width 0.2) (layer "F.Cu") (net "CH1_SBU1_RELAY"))
 (segment (start 28.2111 30.2489) (end 25.73 32.73) (width 0.2) (layer "F.Cu") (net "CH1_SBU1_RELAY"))
 (segment (start 27.7232 36.5239) (end 28.7829 36.5239) (width 0.2) (layer "F.Cu") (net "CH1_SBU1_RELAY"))
 (segment (start 58.9296 25.6016) (end 62.95 25.6016) (width 0.2) (layer "F.Cu") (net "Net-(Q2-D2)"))
 (segment (start 44.9483 34) (end 44.9483 34.6017) (width 0.2) (layer "F.Cu") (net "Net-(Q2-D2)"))
 (segment (start 47.4923 23.794) (end 57.122 23.794) (width 0.2) (layer "F.Cu") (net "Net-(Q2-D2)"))
 (segment (start 44.9483 34.6017) (end 44.8736 34.6764) (width 0.2) (layer "F.Cu") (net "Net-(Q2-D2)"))
 (segment (start 62.95 24.6999) (end 62.95 25.6016) (width 0.2) (layer "F.Cu") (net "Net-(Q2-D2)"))
 (segment (start 57.122 23.794) (end 58.9296 25.6016) (width 0.2) (layer "F.Cu") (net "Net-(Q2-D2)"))
 (segment (start 45.55 34) (end 44.9483 34) (width 0.2) (layer "F.Cu") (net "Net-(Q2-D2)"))
 (via (at 44.8736 34.6764) (size 0.6) (drill 0.3) (layers "F.Cu" "B.Cu") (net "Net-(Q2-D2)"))
 (via (at 47.4923 23.794) (size 0.6) (drill 0.3) (layers "F.Cu" "B.Cu") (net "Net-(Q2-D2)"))
 (segment (start 47.4923 23.794) (end 44.8736 26.4127) (width 0.2) (layer "B.Cu") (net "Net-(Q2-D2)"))
 (segment (start 44.8736 26.4127) (end 44.8736 34.6764) (width 0.2) (layer "B.Cu") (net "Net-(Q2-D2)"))
 (segment (start 46.45 34) (end 47.0517 34) (width 0.2) (layer "F.Cu") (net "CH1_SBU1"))
 (segment (start 28.4801 30.6506) (end 27 32.1307) (width 0.2) (layer "F.Cu") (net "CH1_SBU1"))
 (segment (start 61.45 34.6017) (end 58.5517 37.5) (width 0.2) (layer "F.Cu") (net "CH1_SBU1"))
 (segment (start 27 34) (end 28.27 35.27) (width 0.2) (layer "F.Cu") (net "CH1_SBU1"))
 (segment (start 62.45 42) (end 62.45 41.3983) (width 0.2) (layer "F.Cu") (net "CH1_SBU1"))
 (segment (start 46.45 33.3983) (end 43.7023 30.6506) (width 0.2) (layer "F.Cu") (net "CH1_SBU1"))
 (segment (start 62.45 41.3983) (end 58.5517 37.5) (width 0.2) (layer "F.Cu") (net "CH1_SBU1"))
 (segment (start 50.5517 37.5) (end 47.0517 34) (width 0.2) (layer "F.Cu") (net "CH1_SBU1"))
 (segment (start 58.5517 37.5) (end 50.5517 37.5) (width 0.2) (layer "F.Cu") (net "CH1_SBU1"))
 (segment (start 43.7023 30.6506) (end 28.4801 30.6506) (width 0.2) (layer "F.Cu") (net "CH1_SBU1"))
 (segment (start 27 32.1307) (end 27 34) (width 0.2) (layer "F.Cu") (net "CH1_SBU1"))
 (segment (start 46.45 34) (end 46.45 33.3983) (width 0.2) (layer "F.Cu") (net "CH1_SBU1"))
 (segment (start 61.45 34) (end 61.45 34.6017) (width 0.2) (layer "F.Cu") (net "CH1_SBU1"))
 (segment (start 45.55 50.6017) (end 60.3466 50.6017) (width 0.2) (layer "F.Cu") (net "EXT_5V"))
 (segment (start 30.81 35.27) (end 36.9483 41.4083) (width 0.2) (layer "F.Cu") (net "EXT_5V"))
 (segment (start 37.2492 42) (end 37.1005 42.1487) (width 0.2) (layer "F.Cu") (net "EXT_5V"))
 (segment (start 36.9483 41.4083) (end 36.9483 42) (width 0.2) (layer "F.Cu") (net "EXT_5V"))
 (segment (start 45.55 50) (end 45.55 50.6017) (width 0.2) (layer "F.Cu") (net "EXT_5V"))
 (segment (start 37.55 42) (end 37.2492 42) (width 0.2) (layer "F.Cu") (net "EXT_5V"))
 (segment (start 45.1 42) (end 44.3983 42) (width 0.2) (layer "F.Cu") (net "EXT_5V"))
 (segment (start 44.3983 42) (end 43.7966 41.3983) (width 0.2) (layer "F.Cu") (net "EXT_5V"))
 (segment (start 42.5133 50) (end 45.55 50) (width 0.2) (layer "F.Cu") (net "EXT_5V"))
 (segment (start 37.1005 42.1487) (end 37.1005 44.5872) (width 0.2) (layer "F.Cu") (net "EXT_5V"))
 (segment (start 37.1005 44.5872) (end 42.5133 50) (width 0.2) (layer "F.Cu") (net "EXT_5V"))
 (segment (start 37.2492 42) (end 36.9483 42) (width 0.2) (layer "F.Cu") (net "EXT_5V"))
 (segment (start 60.3466 50.6017) (end 60.9483 50) (width 0.2) (layer "F.Cu") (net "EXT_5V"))
 (segment (start 43.7966 41.3983) (end 36.9583 41.3983) (width 0.2) (layer "F.Cu") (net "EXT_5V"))
 (segment (start 36.9583 41.3983) (end 36.9483 41.4083) (width 0.2) (layer "F.Cu") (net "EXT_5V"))
 (segment (start 61.55 50) (end 60.9483 50) (width 0.2) (layer "F.Cu") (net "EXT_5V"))
 (segment (start 29.54 34) (end 24.46 34) (width 0.2) (layer "B.Cu") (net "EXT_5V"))
 (segment (start 30.81 35.27) (end 29.54 34) (width 0.2) (layer "B.Cu") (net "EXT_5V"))
 (segment (start 24.46 34) (end 23.19 32.73) (width 0.2) (layer "B.Cu") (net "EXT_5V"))
 (segment (start 60.55 34) (end 59.05 34) (width 0.2) (layer "F.Cu") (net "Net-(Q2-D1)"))
 (segment (start 63.5272 30.1443) (end 63.5272 23.9434) (width 0.2) (layer "F.Cu") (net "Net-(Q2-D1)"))
 (segment (start 61.05 24.6999) (end 61.05 23.7982) (width 0.2) (layer "F.Cu") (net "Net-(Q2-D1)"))
 (segment (start 63.5272 23.9434) (end 63.382 23.7982) (width 0.2) (layer "F.Cu") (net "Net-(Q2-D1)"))
 (segment (start 63.382 23.7982) (end 61.05 23.7982) (width 0.2) (layer "F.Cu") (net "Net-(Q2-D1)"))
 (segment (start 60.55 34) (end 60.55 33.1215) (width 0.2) (layer "F.Cu") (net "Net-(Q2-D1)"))
 (segment (start 60.55 33.1215) (end 63.5272 30.1443) (width 0.2) (layer "F.Cu") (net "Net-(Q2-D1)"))
 (via (at 59.05 34) (size 0.6) (drill 0.3) (layers "F.Cu" "B.Cu") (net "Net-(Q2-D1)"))
 (segment (start 59.05 34) (end 58.05 34) (width 0.2) (layer "B.Cu") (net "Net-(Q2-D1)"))
 (segment (start 50.0014 48.1638) (end 48.8879 48.1638) (width 0.2) (layer "F.Cu") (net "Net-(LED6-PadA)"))
 (segment (start 46.45 50) (end 47.0517 50) (width 0.2) (layer "F.Cu") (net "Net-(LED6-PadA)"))
 (segment (start 48.8879 48.1638) (end 47.0517 50) (width 0.2) (layer "F.Cu") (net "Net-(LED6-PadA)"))
 (segment (start 54 27.05) (end 50.5108 27.05) (width 0.2) (layer "F.Cu") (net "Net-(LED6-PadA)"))
 (via (at 50.0014 48.1638) (size 0.6) (drill 0.3) (layers "F.Cu" "B.Cu") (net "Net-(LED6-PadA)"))
 (via (at 50.5108 27.05) (size 0.6) (drill 0.3) (layers "F.Cu" "B.Cu") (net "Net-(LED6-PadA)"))
 (segment (start 50.0014 48.1638) (end 50.5108 47.6544) (width 0.2) (layer "B.Cu") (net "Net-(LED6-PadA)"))
 (segment (start 50.5108 47.6544) (end 50.5108 27.05) (width 0.2) (layer "B.Cu") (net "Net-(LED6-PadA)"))
 (segment (start 45.55 26) (end 30.6578 26) (width 0.2) (layer "F.Cu") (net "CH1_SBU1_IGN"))
 (segment (start 45.55 26) (end 45.55 26.6017) (width 0.2) (layer "F.Cu") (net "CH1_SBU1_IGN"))
 (segment (start 24.46 34) (end 25.73 35.27) (width 0.2) (layer "F.Cu") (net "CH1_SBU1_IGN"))
 (segment (start 24.46 32.1978) (end 24.46 34) (width 0.2) (layer "F.Cu") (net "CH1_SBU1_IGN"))
 (segment (start 30.6578 26) (end 24.46 32.1978) (width 0.2) (layer "F.Cu") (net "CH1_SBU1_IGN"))
 (segment (start 37.7022 44.3381) (end 49.3898 44.3381) (width 0.2) (layer "F.Cu") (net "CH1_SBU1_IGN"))
 (segment (start 61.05 27.3001) (end 61.05 28.2018) (width 0.2) (layer "F.Cu") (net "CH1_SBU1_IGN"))
 (segment (start 61.05 28.2018) (end 47.1501 28.2018) (width 0.2) (layer "F.Cu") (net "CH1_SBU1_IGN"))
 (segment (start 47.1501 28.2018) (end 45.55 26.6017) (width 0.2) (layer "F.Cu") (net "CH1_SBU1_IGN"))
 (segment (start 49.3898 44.3381) (end 54.45 49.3983) (width 0.2) (layer "F.Cu") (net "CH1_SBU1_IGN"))
 (segment (start 54.45 50) (end 54.45 49.3983) (width 0.2) (layer "F.Cu") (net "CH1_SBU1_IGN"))
 (via (at 37.7022 44.3381) (size 0.6) (drill 0.3) (layers "F.Cu" "B.Cu") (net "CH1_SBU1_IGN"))
 (segment (start 34.7981 44.3381) (end 37.7022 44.3381) (width 0.2) (layer "B.Cu") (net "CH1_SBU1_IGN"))
 (segment (start 25.73 35.27) (end 34.7981 44.3381) (width 0.2) (layer "B.Cu") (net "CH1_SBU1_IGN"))
 (segment (start 61.55 42) (end 48.864 42) (width 0.2) (layer "F.Cu") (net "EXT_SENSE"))
 (segment (start 48.864 42) (end 37.9163 31.0523) (width 0.2) (layer "F.Cu") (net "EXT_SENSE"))
 (segment (start 37.9163 31.0523) (end 29.9477 31.0523) (width 0.2) (layer "F.Cu") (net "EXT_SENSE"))
 (segment (start 29.9477 31.0523) (end 28.27 32.73) (width 0.2) (layer "F.Cu") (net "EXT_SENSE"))
 (segment (start 37.8298 27.0781) (end 37.9568 27.0781) (width 0.2) (layer "F.Cu") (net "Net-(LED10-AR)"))
 (segment (start 53.55 50) (end 52.9483 50) (width 0.2) (layer "F.Cu") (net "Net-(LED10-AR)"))
 (segment (start 49.4697 46.5214) (end 52.9483 50) (width 0.2) (layer "F.Cu") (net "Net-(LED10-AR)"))
 (segment (start 37.05 27) (end 37.7517 27) (width 0.2) (layer "F.Cu") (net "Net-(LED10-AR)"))
 (segment (start 40.3947 46.5214) (end 49.4697 46.5214) (width 0.2) (layer "F.Cu") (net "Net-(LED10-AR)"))
 (segment (start 37.7517 27) (end 37.8298 27.0781) (width 0.2) (layer "F.Cu") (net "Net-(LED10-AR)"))
 (via (at 37.9568 27.0781) (size 0.6) (drill 0.3) (layers "F.Cu" "B.Cu") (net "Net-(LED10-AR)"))
 (via (at 40.3947 46.5214) (size 0.6) (drill 0.3) (layers "F.Cu" "B.Cu") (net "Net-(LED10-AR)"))
 (segment (start 40.3947 46.5214) (end 40.3947 29.516) (width 0.2) (layer "B.Cu") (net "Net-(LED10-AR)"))
 (segment (start 40.3947 29.516) (end 37.9568 27.0781) (width 0.2) (layer "B.Cu") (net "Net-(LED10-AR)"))
 (segment (start 53.55 34) (end 52.9483 34) (width 0.2) (layer "F.Cu") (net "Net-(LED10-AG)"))
 (segment (start 38.95 27) (end 39.6517 27) (width 0.2) (layer "F.Cu") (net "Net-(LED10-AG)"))
 (segment (start 43.0846 27) (end 39.6517 27) (width 0.2) (layer "F.Cu") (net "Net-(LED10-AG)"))
 (segment (start 50.0846 34) (end 43.0846 27) (width 0.2) (layer "F.Cu") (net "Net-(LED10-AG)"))
 (segment (start 52.9483 34) (end 50.0846 34) (width 0.2) (layer "F.Cu") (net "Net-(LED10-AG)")))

